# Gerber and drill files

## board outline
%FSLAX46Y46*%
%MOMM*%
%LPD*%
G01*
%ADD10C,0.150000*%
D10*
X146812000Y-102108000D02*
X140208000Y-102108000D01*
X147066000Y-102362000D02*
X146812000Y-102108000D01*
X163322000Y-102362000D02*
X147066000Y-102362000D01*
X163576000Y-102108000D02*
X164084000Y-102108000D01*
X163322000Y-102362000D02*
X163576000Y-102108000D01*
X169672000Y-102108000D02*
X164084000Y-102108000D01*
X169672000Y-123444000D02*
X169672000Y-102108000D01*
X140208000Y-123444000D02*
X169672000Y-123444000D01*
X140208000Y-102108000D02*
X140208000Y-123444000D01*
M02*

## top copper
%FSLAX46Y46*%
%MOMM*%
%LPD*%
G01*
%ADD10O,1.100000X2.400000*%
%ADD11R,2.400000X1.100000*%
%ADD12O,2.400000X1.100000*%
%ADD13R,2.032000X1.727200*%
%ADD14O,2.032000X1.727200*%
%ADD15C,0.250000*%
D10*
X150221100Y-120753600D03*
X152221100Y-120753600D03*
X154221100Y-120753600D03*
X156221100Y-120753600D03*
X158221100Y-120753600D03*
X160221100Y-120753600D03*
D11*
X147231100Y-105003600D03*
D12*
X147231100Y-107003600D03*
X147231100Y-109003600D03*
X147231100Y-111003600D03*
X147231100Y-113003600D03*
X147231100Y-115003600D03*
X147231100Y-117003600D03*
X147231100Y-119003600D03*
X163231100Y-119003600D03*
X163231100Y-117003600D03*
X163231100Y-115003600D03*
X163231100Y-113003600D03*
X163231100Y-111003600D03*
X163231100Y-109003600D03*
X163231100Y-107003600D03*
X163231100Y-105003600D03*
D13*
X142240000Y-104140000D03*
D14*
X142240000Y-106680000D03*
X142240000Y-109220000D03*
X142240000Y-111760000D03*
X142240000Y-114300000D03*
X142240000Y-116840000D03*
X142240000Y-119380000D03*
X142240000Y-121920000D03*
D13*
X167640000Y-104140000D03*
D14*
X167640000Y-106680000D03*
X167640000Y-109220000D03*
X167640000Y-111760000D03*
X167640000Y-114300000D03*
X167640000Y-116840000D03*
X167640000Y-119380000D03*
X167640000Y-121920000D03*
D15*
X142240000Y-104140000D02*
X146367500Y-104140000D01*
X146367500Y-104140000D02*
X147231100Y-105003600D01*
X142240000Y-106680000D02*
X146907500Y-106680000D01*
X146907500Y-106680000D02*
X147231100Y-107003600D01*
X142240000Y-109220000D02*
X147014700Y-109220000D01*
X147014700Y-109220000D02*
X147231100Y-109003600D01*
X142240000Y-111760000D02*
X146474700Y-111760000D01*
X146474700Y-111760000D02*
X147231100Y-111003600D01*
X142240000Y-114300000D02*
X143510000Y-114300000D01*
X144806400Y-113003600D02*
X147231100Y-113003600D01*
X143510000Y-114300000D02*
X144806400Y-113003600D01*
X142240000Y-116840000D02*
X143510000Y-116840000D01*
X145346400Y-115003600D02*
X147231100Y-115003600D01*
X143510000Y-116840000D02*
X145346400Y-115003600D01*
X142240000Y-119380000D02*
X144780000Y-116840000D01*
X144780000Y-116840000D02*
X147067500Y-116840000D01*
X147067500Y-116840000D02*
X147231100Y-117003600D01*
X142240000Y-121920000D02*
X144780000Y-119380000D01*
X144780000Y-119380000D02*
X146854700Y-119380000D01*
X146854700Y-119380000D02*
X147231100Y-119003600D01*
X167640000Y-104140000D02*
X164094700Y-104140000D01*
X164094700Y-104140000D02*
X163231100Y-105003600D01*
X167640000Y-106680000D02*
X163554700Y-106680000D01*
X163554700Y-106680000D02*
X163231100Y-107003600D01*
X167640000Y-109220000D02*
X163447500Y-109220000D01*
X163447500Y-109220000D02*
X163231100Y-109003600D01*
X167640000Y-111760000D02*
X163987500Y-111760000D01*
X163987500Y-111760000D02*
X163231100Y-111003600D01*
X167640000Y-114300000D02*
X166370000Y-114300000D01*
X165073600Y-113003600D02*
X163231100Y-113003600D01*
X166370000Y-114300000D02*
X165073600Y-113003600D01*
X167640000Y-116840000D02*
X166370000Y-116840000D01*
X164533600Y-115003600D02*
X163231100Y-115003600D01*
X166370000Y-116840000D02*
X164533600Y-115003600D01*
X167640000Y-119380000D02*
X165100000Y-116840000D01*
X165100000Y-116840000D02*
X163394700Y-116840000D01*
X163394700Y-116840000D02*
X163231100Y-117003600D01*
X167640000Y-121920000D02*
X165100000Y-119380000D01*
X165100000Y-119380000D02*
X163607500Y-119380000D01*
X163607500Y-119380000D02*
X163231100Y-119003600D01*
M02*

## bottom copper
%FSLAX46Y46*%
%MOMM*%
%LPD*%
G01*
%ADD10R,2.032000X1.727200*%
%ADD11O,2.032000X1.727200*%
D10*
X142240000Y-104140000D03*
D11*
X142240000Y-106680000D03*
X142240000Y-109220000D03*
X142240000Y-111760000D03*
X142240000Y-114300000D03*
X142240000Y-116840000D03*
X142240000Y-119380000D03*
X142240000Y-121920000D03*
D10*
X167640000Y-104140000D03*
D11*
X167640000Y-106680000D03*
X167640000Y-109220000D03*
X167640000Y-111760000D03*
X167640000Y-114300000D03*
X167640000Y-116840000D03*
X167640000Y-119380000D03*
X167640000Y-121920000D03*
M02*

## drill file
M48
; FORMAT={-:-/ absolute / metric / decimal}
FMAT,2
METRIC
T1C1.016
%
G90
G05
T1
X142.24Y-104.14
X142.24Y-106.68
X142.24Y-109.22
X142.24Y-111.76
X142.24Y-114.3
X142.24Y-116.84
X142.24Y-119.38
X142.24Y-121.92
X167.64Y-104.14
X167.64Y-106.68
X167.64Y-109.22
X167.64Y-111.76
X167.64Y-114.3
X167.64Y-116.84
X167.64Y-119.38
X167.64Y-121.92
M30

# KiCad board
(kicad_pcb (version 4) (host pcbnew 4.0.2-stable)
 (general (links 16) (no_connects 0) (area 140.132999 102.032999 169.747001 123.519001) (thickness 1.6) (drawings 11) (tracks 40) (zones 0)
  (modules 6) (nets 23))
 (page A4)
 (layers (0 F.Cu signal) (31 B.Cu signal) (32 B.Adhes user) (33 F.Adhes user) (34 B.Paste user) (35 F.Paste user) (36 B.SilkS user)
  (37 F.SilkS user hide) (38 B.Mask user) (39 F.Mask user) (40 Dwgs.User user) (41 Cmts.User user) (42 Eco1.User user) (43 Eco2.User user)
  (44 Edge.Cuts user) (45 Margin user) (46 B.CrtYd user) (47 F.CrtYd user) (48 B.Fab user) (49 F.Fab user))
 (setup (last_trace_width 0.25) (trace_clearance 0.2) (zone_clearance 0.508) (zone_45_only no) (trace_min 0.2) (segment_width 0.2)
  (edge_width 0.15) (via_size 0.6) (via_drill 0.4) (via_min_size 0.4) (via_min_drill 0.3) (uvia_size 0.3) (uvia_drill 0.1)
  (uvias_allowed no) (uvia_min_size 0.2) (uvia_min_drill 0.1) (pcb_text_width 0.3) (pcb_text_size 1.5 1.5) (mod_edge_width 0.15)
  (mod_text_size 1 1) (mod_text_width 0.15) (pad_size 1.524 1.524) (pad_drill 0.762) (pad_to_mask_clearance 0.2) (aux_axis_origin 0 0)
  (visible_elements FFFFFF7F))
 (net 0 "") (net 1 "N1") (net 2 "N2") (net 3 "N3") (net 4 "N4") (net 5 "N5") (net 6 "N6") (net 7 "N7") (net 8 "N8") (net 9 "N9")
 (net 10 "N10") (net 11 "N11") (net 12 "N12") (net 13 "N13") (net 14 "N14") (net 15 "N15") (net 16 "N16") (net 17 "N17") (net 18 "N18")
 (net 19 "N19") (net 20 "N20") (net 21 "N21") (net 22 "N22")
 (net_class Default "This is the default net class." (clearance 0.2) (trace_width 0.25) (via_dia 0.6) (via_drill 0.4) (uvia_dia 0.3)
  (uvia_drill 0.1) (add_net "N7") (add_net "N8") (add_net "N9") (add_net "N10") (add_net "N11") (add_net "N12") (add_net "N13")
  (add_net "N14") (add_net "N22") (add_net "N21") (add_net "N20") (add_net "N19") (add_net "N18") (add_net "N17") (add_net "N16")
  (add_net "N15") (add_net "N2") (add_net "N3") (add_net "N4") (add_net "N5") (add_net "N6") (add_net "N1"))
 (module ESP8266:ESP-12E (layer F.Cu) (at 147.2311 105.0036)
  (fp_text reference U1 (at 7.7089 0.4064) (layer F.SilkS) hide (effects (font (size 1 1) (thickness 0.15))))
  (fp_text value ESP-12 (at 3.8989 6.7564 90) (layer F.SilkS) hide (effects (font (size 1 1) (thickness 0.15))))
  (pad 9 smd oval (at 2.99 15.75 90) (size 2.4 1.1) (layers F.Cu F.Paste F.Mask) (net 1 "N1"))
  (pad 10 smd oval (at 4.99 15.75 90) (size 2.4 1.1) (layers F.Cu F.Paste F.Mask) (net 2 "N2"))
  (pad 11 smd oval (at 6.99 15.75 90) (size 2.4 1.1) (layers F.Cu F.Paste F.Mask) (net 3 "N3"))
  (pad 12 smd oval (at 8.99 15.75 90) (size 2.4 1.1) (layers F.Cu F.Paste F.Mask) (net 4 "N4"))
  (pad 13 smd oval (at 10.99 15.75 90) (size 2.4 1.1) (layers F.Cu F.Paste F.Mask) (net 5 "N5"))
  (pad 14 smd oval (at 12.99 15.75 90) (size 2.4 1.1) (layers F.Cu F.Paste F.Mask) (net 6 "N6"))
  (pad 1 smd rect (at 0 0) (size 2.4 1.1) (layers F.Cu F.Paste F.Mask) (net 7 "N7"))
  (pad 2 smd oval (at 0 2) (size 2.4 1.1) (layers F.Cu F.Paste F.Mask) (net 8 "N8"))
  (pad 3 smd oval (at 0 4) (size 2.4 1.1) (layers F.Cu F.Paste F.Mask) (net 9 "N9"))
  (pad 4 smd oval (at 0 6) (size 2.4 1.1) (layers F.Cu F.Paste F.Mask) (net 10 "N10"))
  (pad 5 smd oval (at 0 8) (size 2.4 1.1) (layers F.Cu F.Paste F.Mask) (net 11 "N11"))
  (pad 6 smd oval (at 0 10) (size 2.4 1.1) (layers F.Cu F.Paste F.Mask) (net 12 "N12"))
  (pad 7 smd oval (at 0 12) (size 2.4 1.1) (layers F.Cu F.Paste F.Mask) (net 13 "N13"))
  (pad 8 smd oval (at 0 14) (size 2.4 1.1) (layers F.Cu F.Paste F.Mask) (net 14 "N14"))
  (pad 15 smd oval (at 16 14) (size 2.4 1.1) (layers F.Cu F.Paste F.Mask) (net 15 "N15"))
  (pad 16 smd oval (at 16 12) (size 2.4 1.1) (layers F.Cu F.Paste F.Mask) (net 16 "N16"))
  (pad 17 smd oval (at 16 10) (size 2.4 1.1) (layers F.Cu F.Paste F.Mask) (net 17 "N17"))
  (pad 18 smd oval (at 16 8) (size 2.4 1.1) (layers F.Cu F.Paste F.Mask) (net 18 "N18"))
  (pad 19 smd oval (at 16 6) (size 2.4 1.1) (layers F.Cu F.Paste F.Mask) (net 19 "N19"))
  (pad 20 smd oval (at 16 4) (size 2.4 1.1) (layers F.Cu F.Paste F.Mask) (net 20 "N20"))
  (pad 21 smd oval (at 16 2) (size 2.4 1.1) (layers F.Cu F.Paste F.Mask) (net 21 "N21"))
  (pad 22 smd oval (at 16 0) (size 2.4 1.1) (layers F.Cu F.Paste F.Mask) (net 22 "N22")))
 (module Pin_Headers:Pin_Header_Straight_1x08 (layer F.Cu) (at 142.24 104.14)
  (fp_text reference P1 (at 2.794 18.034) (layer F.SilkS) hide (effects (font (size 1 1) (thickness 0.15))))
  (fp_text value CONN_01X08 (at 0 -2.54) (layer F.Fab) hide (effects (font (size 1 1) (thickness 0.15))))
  (pad 1 thru_hole rect (at 0 0) (size 2.032 1.7272) (drill 1.016) (layers *.Cu *.Mask F.SilkS) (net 7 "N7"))
  (pad 2 thru_hole oval (at 0 2.54) (size 2.032 1.7272) (drill 1.016) (layers *.Cu *.Mask F.SilkS) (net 8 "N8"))
  (pad 3 thru_hole oval (at 0 5.08) (size 2.032 1.7272) (drill 1.016) (layers *.Cu *.Mask F.SilkS) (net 9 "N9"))
  (pad 4 thru_hole oval (at 0 7.62) (size 2.032 1.7272) (drill 1.016) (layers *.Cu *.Mask F.SilkS) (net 10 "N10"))
  (pad 5 thru_hole oval (at 0 10.16) (size 2.032 1.7272) (drill 1.016) (layers *.Cu *.Mask F.SilkS) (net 11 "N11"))
  (pad 6 thru_hole oval (at 0 12.7) (size 2.032 1.7272) (drill 1.016) (layers *.Cu *.Mask F.SilkS) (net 12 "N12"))
  (pad 7 thru_hole oval (at 0 15.24) (size 2.032 1.7272) (drill 1.016) (layers *.Cu *.Mask F.SilkS) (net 13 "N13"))
  (pad 8 thru_hole oval (at 0 17.78) (size 2.032 1.7272) (drill 1.016) (layers *.Cu *.Mask F.SilkS) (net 14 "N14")))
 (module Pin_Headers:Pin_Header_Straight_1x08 (layer F.Cu) (at 167.64 104.14)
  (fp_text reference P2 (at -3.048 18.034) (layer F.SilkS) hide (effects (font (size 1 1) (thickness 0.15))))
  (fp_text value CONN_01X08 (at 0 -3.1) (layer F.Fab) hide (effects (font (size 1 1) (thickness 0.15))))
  (pad 1 thru_hole rect (at 0 0) (size 2.032 1.7272) (drill 1.016) (layers *.Cu *.Mask F.SilkS) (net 22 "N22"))
  (pad 2 thru_hole oval (at 0 2.54) (size 2.032 1.7272) (drill 1.016) (layers *.Cu *.Mask F.SilkS) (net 21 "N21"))
  (pad 3 thru_hole oval (at 0 5.08) (size 2.032 1.7272) (drill 1.016) (layers *.Cu *.Mask F.SilkS) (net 20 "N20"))
  (pad 4 thru_hole oval (at 0 7.62) (size 2.032 1.7272) (drill 1.016) (layers *.Cu *.Mask F.SilkS) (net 19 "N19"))
  (pad 5 thru_hole oval (at 0 10.16) (size 2.032 1.7272) (drill 1.016) (layers *.Cu *.Mask F.SilkS) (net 18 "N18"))
  (pad 6 thru_hole oval (at 0 12.7) (size 2.032 1.7272) (drill 1.016) (layers *.Cu *.Mask F.SilkS) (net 17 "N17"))
  (pad 7 thru_hole oval (at 0 15.24) (size 2.032 1.7272) (drill 1.016) (layers *.Cu *.Mask F.SilkS) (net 16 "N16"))
  (pad 8 thru_hole oval (at 0 17.78) (size 2.032 1.7272) (drill 1.016) (layers *.Cu *.Mask F.SilkS) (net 15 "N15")))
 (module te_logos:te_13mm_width (layer F.Cu) (at 159.258 111.506 90)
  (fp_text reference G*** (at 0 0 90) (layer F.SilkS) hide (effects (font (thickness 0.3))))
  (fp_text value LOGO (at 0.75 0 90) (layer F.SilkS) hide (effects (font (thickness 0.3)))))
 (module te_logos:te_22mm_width (layer B.Cu) (at 154.94 117.094 180)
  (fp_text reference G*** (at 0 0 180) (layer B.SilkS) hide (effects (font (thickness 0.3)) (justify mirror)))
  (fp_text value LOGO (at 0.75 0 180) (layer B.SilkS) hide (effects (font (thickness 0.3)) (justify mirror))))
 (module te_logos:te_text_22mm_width (layer B.Cu) (at 154.94 120.904 180)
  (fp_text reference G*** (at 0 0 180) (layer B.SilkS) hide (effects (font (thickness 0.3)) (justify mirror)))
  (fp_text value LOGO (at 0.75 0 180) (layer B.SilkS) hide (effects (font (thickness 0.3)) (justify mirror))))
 (gr_line (start 146.812 102.108) (end 140.208 102.108) (angle 90) (layer Edge.Cuts) (width 0.15))
 (gr_line (start 147.066 102.362) (end 146.812 102.108) (angle 90) (layer Edge.Cuts) (width 0.15))
 (gr_line (start 163.322 102.362) (end 147.066 102.362) (angle 90) (layer Edge.Cuts) (width 0.15))
 (gr_line (start 163.576 102.108) (end 164.084 102.108) (angle 90) (layer Edge.Cuts) (width 0.15))
 (gr_line (start 163.322 102.362) (end 163.576 102.108) (angle 90) (layer Edge.Cuts) (width 0.15))
 (gr_line (start 169.672 102.108) (end 164.084 102.108) (angle 90) (layer Edge.Cuts) (width 0.15))
 (gr_line (start 169.672 123.444) (end 169.672 102.108) (angle 90) (layer Edge.Cuts) (width 0.15))
 (gr_line (start 140.208 123.444) (end 169.672 123.444) (angle 90) (layer Edge.Cuts) (width 0.15))
 (gr_line (start 140.208 102.108) (end 140.208 123.444) (angle 90) (layer Edge.Cuts) (width 0.15))
 (segment (start 142.24 104.14) (end 146.3675 104.14) (width 0.25) (layer F.Cu) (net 7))
 (segment (start 146.3675 104.14) (end 147.2311 105.0036) (width 0.25) (layer F.Cu) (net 7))
 (segment (start 142.24 106.68) (end 146.9075 106.68) (width 0.25) (layer F.Cu) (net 8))
 (segment (start 146.9075 106.68) (end 147.2311 107.0036) (width 0.25) (layer F.Cu) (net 8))
 (segment (start 142.24 109.22) (end 147.0147 109.22) (width 0.25) (layer F.Cu) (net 9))
 (segment (start 147.0147 109.22) (end 147.2311 109.0036) (width 0.25) (layer F.Cu) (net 9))
 (segment (start 142.24 111.76) (end 146.4747 111.76) (width 0.25) (layer F.Cu) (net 10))
 (segment (start 146.4747 111.76) (end 147.2311 111.0036) (width 0.25) (layer F.Cu) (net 10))
 (segment (start 142.24 114.3) (end 143.51 114.3) (width 0.25) (layer F.Cu) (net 11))
 (segment (start 144.8064 113.0036) (end 147.2311 113.0036) (width 0.25) (layer F.Cu) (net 11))
 (segment (start 143.51 114.3) (end 144.8064 113.0036) (width 0.25) (layer F.Cu) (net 11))
 (segment (start 142.24 116.84) (end 143.51 116.84) (width 0.25) (layer F.Cu) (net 12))
 (segment (start 145.3464 115.0036) (end 147.2311 115.0036) (width 0.25) (layer F.Cu) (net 12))
 (segment (start 143.51 116.84) (end 145.3464 115.0036) (width 0.25) (layer F.Cu) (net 12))
 (segment (start 142.24 119.38) (end 144.78 116.84) (width 0.25) (layer F.Cu) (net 13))
 (segment (start 144.78 116.84) (end 147.0675 116.84) (width 0.25) (layer F.Cu) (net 13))
 (segment (start 147.0675 116.84) (end 147.2311 117.0036) (width 0.25) (layer F.Cu) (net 13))
 (segment (start 142.24 121.92) (end 144.78 119.38) (width 0.25) (layer F.Cu) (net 14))
 (segment (start 144.78 119.38) (end 146.8547 119.38) (width 0.25) (layer F.Cu) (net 14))
 (segment (start 146.8547 119.38) (end 147.2311 119.0036) (width 0.25) (layer F.Cu) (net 14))
 (segment (start 167.64 104.14) (end 164.0947 104.14) (width 0.25) (layer F.Cu) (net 22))
 (segment (start 164.0947 104.14) (end 163.2311 105.0036) (width 0.25) (layer F.Cu) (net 22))
 (segment (start 167.64 106.68) (end 163.5547 106.68) (width 0.25) (layer F.Cu) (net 21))
 (segment (start 163.5547 106.68) (end 163.2311 107.0036) (width 0.25) (layer F.Cu) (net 21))
 (segment (start 167.64 109.22) (end 163.4475 109.22) (width 0.25) (layer F.Cu) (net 20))
 (segment (start 163.4475 109.22) (end 163.2311 109.0036) (width 0.25) (layer F.Cu) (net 20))
 (segment (start 167.64 111.76) (end 163.9875 111.76) (width 0.25) (layer F.Cu) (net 19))
 (segment (start 163.9875 111.76) (end 163.2311 111.0036) (width 0.25) (layer F.Cu) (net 19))
 (segment (start 167.64 114.3) (end 166.37 114.3) (width 0.25) (layer F.Cu) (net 18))
 (segment (start 165.0736 113.0036) (end 163.2311 113.0036) (width 0.25) (layer F.Cu) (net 18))
 (segment (start 166.37 114.3) (end 165.0736 113.0036) (width 0.25) (layer F.Cu) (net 18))
 (segment (start 167.64 116.84) (end 166.37 116.84) (width 0.25) (layer F.Cu) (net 17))
 (segment (start 164.5336 115.0036) (end 163.2311 115.0036) (width 0.25) (layer F.Cu) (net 17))
 (segment (start 166.37 116.84) (end 164.5336 115.0036) (width 0.25) (layer F.Cu) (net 17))
 (segment (start 167.64 119.38) (end 165.1 116.84) (width 0.25) (layer F.Cu) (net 16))
 (segment (start 165.1 116.84) (end 163.3947 116.84) (width 0.25) (layer F.Cu) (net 16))
 (segment (start 163.3947 116.84) (end 163.2311 117.0036) (width 0.25) (layer F.Cu) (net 16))
 (segment (start 167.64 121.92) (end 165.1 119.38) (width 0.25) (layer F.Cu) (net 15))
 (segment (start 165.1 119.38) (end 163.6075 119.38) (width 0.25) (layer F.Cu) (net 15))
 (segment (start 163.6075 119.38) (end 163.2311 119.0036) (width 0.25) (layer F.Cu) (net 15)))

